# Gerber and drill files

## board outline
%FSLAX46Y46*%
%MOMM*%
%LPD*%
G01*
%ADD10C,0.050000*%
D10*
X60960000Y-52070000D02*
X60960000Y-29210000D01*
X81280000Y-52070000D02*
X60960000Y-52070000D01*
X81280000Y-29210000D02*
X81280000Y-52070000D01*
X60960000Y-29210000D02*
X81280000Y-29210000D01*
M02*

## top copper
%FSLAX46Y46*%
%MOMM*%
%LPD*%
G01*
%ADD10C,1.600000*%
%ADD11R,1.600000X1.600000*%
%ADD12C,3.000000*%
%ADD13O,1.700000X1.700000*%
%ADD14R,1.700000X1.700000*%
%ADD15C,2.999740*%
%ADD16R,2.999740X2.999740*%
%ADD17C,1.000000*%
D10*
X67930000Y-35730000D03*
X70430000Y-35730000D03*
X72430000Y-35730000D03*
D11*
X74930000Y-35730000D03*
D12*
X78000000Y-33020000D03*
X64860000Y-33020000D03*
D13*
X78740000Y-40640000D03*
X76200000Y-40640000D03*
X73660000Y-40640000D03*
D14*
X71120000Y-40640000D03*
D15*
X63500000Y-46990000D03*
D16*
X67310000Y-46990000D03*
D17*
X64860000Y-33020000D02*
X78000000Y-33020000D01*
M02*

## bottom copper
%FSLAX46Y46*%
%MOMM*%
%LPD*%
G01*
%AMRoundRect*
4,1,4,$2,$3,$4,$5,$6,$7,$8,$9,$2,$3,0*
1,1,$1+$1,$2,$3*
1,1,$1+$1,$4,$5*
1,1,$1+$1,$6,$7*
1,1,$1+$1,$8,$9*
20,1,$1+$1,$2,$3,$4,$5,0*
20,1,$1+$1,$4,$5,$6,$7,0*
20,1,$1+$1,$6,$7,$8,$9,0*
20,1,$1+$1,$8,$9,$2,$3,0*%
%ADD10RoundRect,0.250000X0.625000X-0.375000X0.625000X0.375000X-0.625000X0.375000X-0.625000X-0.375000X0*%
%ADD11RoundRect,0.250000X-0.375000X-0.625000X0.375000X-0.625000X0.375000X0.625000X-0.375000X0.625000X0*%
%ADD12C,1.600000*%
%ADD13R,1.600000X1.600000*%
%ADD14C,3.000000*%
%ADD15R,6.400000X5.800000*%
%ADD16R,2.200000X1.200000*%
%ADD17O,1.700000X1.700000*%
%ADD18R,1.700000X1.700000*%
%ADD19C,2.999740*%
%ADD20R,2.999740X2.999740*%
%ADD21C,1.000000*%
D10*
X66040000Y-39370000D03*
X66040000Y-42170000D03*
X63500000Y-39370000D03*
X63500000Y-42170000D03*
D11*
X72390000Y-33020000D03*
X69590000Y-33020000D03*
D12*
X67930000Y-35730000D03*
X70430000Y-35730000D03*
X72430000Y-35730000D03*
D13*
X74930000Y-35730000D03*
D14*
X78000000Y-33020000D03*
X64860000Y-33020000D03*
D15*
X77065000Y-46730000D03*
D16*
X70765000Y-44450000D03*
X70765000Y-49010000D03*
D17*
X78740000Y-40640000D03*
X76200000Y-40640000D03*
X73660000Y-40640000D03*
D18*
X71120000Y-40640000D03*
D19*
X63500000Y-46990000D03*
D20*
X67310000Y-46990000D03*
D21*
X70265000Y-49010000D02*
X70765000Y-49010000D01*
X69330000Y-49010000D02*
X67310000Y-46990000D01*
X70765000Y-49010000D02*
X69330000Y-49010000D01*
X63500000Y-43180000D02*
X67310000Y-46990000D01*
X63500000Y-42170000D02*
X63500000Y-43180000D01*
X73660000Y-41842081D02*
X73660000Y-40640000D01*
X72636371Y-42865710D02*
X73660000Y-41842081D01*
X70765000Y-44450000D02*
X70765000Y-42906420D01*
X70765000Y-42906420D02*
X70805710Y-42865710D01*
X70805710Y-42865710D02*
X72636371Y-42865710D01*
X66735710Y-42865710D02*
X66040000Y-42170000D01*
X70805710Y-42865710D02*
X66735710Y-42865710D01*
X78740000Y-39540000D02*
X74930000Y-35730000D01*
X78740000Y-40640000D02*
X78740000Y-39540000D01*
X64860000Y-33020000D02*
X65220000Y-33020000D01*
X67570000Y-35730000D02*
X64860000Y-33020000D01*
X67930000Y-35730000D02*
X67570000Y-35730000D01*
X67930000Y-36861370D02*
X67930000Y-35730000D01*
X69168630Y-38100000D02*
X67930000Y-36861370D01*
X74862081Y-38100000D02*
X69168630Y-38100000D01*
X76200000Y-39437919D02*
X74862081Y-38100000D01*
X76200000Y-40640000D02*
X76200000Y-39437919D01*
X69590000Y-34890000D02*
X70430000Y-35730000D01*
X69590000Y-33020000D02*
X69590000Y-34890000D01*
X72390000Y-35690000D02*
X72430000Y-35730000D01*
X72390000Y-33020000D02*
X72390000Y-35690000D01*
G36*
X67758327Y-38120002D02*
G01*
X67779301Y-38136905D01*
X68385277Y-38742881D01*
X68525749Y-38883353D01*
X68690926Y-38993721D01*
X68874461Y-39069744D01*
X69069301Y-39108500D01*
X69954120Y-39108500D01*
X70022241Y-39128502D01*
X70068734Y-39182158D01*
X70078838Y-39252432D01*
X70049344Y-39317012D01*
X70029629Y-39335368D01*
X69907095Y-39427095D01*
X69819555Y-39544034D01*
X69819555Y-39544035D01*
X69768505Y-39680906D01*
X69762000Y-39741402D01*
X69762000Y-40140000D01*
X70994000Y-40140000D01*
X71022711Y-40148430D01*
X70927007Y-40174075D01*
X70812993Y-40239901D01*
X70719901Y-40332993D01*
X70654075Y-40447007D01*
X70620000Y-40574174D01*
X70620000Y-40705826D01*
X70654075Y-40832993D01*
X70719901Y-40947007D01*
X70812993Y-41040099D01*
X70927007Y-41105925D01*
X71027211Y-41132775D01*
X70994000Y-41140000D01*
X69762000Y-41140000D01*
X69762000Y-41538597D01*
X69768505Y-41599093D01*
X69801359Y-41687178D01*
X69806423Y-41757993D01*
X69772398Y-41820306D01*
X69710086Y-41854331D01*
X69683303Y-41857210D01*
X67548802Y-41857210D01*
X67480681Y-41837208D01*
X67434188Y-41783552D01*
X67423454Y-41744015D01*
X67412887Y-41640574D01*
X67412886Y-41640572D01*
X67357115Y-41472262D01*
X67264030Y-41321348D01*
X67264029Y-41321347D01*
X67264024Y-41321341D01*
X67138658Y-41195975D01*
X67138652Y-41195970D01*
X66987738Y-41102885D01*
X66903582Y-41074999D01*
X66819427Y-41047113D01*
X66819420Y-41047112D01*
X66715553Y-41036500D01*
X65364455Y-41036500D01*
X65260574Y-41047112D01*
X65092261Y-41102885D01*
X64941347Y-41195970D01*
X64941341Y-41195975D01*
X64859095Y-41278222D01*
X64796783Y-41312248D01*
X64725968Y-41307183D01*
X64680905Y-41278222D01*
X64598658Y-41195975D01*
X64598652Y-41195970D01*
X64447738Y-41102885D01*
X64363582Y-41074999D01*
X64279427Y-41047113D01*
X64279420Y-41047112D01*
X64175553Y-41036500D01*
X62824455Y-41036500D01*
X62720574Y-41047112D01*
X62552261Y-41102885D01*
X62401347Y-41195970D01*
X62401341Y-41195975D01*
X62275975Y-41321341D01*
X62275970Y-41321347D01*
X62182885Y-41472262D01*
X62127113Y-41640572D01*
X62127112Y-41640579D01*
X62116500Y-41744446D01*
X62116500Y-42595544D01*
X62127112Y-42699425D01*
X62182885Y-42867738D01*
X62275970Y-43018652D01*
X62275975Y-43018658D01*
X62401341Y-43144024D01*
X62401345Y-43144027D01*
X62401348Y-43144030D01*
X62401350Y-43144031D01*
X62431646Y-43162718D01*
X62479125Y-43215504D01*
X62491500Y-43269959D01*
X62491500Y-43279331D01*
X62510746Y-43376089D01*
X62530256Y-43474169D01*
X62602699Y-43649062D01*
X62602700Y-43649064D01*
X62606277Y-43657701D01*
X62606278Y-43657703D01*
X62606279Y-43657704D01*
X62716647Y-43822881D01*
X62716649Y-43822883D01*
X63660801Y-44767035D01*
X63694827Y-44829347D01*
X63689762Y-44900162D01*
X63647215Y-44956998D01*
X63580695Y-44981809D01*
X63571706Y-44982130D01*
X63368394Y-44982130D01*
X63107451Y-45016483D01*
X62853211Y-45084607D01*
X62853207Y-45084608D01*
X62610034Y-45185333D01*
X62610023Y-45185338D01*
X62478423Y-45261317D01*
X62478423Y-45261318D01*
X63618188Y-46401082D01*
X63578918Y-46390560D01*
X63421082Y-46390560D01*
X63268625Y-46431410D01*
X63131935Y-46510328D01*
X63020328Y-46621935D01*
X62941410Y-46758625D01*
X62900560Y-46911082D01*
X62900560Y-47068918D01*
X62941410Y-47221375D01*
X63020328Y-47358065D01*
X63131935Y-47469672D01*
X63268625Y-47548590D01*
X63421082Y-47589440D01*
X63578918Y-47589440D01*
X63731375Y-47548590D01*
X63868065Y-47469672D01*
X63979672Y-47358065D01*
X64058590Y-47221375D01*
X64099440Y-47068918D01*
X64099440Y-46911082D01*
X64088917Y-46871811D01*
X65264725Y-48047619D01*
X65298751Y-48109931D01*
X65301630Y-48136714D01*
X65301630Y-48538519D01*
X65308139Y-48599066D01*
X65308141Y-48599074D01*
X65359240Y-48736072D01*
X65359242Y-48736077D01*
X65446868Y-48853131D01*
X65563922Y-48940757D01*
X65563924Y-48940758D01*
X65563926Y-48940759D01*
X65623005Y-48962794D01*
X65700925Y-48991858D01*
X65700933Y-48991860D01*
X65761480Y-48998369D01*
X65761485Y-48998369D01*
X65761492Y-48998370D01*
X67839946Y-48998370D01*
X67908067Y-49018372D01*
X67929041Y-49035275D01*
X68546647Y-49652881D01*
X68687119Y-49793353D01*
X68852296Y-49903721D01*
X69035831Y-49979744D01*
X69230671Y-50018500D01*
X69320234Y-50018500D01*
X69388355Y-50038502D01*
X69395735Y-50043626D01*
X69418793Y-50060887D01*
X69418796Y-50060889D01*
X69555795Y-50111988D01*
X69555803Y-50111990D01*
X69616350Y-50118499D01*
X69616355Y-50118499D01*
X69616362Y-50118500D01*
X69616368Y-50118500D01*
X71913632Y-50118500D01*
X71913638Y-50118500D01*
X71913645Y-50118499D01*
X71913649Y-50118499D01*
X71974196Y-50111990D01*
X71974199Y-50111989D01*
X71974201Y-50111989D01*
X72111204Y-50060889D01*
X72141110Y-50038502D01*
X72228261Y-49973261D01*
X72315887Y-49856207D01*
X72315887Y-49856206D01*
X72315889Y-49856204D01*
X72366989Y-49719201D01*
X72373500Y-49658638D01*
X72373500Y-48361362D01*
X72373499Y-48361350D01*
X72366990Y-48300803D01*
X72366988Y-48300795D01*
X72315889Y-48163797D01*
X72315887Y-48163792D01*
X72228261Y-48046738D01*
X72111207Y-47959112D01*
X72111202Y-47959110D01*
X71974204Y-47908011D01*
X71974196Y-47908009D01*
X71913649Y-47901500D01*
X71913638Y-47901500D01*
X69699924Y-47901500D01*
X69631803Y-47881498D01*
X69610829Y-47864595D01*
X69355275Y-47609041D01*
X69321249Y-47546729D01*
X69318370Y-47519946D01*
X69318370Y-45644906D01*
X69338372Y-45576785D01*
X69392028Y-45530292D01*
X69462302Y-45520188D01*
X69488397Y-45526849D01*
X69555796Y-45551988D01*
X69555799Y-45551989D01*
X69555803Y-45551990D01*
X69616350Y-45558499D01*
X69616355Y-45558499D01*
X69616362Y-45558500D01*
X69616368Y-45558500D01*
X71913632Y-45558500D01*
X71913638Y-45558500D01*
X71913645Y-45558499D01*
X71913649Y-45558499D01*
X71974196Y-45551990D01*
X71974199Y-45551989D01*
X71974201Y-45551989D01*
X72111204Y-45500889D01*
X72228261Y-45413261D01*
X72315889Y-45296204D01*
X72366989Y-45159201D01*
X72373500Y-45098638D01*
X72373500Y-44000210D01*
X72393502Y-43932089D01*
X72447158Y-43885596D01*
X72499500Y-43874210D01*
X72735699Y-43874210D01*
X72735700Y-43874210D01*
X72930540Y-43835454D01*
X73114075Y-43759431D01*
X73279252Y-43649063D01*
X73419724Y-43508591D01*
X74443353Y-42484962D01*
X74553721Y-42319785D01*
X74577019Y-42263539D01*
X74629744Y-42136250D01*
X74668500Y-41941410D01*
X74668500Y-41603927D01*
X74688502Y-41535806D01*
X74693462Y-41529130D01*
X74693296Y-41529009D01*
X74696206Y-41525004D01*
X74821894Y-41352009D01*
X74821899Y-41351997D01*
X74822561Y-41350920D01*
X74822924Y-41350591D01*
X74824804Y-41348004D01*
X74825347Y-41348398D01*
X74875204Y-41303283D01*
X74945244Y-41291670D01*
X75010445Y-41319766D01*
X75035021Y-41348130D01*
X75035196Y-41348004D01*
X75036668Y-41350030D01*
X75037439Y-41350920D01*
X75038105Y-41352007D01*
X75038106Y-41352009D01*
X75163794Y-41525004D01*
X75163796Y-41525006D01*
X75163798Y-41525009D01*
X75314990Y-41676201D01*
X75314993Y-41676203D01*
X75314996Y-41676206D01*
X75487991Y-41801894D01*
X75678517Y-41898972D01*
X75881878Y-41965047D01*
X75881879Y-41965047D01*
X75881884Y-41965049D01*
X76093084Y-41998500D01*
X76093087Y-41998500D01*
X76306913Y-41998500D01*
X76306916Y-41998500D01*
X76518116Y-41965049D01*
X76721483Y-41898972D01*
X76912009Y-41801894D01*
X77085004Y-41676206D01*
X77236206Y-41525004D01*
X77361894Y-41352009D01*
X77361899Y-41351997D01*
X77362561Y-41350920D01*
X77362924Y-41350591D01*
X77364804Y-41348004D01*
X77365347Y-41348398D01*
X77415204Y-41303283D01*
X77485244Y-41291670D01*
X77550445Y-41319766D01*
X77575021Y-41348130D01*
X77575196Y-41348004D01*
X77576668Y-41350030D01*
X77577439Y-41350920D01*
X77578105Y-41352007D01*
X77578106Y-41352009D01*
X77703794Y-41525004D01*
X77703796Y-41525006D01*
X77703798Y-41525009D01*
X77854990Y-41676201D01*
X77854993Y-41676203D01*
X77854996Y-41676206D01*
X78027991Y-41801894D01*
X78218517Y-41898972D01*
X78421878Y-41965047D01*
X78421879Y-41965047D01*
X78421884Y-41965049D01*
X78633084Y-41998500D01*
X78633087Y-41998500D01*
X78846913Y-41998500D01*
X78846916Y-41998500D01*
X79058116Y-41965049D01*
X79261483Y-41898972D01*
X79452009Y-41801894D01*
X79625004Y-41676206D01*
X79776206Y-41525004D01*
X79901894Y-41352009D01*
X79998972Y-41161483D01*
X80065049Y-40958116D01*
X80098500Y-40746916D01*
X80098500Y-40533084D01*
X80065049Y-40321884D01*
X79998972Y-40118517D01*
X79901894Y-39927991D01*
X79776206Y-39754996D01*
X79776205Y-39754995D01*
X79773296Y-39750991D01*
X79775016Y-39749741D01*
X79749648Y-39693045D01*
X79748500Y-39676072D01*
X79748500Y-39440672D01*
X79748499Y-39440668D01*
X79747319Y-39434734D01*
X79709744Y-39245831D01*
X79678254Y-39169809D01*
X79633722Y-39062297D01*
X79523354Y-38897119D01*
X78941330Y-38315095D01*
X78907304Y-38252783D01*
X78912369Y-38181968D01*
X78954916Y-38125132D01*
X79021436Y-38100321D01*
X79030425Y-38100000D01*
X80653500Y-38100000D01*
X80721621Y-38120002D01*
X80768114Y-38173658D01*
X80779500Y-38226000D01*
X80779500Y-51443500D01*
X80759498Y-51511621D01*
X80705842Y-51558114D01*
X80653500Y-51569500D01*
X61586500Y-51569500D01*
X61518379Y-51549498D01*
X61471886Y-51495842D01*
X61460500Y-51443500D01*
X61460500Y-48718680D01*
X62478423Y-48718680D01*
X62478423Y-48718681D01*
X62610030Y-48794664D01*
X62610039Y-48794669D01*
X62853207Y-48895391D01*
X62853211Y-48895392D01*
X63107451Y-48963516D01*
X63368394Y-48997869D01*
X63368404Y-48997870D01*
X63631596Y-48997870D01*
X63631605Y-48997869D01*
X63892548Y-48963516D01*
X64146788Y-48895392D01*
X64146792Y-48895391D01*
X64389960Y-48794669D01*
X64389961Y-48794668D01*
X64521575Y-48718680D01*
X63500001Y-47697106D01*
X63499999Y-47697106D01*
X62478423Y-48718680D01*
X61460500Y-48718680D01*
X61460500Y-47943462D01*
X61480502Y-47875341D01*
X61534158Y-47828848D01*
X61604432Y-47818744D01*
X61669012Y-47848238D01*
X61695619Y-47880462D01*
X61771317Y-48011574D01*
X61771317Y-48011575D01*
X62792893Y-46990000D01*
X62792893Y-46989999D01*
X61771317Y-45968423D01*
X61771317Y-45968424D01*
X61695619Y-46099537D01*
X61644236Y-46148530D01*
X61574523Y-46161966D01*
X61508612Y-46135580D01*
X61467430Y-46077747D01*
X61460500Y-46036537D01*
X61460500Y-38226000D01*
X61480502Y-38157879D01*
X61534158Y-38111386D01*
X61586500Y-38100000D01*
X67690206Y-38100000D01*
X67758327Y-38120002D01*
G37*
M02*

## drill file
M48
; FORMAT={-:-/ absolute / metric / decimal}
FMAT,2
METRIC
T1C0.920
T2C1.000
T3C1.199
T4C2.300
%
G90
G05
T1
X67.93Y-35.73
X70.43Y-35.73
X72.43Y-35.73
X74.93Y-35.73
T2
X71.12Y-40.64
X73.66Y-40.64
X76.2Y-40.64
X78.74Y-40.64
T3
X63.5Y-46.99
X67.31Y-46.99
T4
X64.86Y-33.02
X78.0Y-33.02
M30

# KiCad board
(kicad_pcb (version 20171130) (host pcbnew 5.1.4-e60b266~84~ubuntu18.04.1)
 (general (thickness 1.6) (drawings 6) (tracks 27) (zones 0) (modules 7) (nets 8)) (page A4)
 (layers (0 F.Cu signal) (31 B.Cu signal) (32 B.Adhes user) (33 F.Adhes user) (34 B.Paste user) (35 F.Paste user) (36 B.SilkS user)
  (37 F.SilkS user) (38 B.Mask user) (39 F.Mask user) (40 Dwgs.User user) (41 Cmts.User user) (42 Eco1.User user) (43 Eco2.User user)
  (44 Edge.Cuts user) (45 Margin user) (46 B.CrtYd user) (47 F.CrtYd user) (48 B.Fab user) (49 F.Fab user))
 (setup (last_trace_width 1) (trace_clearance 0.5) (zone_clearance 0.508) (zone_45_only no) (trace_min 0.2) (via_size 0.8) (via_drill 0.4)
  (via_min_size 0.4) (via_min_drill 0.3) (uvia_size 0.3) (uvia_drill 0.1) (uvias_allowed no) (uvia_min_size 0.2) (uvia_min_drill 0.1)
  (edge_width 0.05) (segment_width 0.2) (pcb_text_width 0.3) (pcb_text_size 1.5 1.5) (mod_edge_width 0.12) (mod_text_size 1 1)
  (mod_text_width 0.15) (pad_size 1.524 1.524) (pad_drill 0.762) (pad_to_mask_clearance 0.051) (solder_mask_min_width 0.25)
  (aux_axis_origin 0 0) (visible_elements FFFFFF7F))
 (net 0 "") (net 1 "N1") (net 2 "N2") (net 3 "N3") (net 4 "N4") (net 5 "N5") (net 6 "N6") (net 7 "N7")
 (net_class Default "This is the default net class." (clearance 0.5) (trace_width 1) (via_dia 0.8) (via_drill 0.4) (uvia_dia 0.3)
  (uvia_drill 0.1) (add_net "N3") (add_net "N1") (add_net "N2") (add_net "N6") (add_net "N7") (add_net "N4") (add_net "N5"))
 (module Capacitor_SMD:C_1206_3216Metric (layer B.Cu) (at 66.04 40.77 90)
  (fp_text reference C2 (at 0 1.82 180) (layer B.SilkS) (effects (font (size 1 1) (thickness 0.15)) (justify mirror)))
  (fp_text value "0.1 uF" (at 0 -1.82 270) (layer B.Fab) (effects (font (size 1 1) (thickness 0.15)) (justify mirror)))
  (pad 2 smd roundrect (at 1.4 0 90) (size 1.25 1.75) (layers B.Cu B.Paste B.Mask) (roundrect_rratio 0.2) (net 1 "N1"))
  (pad 1 smd roundrect (at -1.4 0 90) (size 1.25 1.75) (layers B.Cu B.Paste B.Mask) (roundrect_rratio 0.2) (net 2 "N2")))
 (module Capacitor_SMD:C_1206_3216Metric (layer B.Cu) (at 63.5 40.77 90)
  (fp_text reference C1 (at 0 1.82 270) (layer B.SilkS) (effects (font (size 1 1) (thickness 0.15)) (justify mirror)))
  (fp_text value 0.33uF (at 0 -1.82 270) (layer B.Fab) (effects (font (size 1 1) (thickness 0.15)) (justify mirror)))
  (pad 2 smd roundrect (at 1.4 0 90) (size 1.25 1.75) (layers B.Cu B.Paste B.Mask) (roundrect_rratio 0.2) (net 1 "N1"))
  (pad 1 smd roundrect (at -1.4 0 90) (size 1.25 1.75) (layers B.Cu B.Paste B.Mask) (roundrect_rratio 0.2) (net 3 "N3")))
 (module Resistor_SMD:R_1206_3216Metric (layer B.Cu) (at 70.99 33.02)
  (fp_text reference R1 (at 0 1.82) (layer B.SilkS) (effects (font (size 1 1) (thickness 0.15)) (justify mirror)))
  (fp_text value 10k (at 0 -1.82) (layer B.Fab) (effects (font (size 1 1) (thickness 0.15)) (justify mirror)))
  (pad 2 smd roundrect (at 1.4 0) (size 1.25 1.75) (layers B.Cu B.Paste B.Mask) (roundrect_rratio 0.2) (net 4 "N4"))
  (pad 1 smd roundrect (at -1.4 0) (size 1.25 1.75) (layers B.Cu B.Paste B.Mask) (roundrect_rratio 0.2) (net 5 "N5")))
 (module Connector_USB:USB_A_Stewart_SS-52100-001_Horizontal (layer F.Cu) (at 74.93 35.73 180)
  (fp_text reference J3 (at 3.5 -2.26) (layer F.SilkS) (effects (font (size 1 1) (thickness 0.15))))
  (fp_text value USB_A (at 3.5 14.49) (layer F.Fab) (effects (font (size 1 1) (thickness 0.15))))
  (pad 4 thru_hole circle (at 7 0 180) (size 1.6 1.6) (drill 0.92) (layers *.Cu *.Mask) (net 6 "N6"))
  (pad 3 thru_hole circle (at 4.5 0 180) (size 1.6 1.6) (drill 0.92) (layers *.Cu *.Mask) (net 5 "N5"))
  (pad 2 thru_hole circle (at 2.5 0 180) (size 1.6 1.6) (drill 0.92) (layers *.Cu *.Mask) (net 4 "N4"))
  (pad 1 thru_hole rect (at 0 0 180) (size 1.6 1.6) (drill 0.92) (layers *.Cu *.Mask) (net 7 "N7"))
  (pad 5 thru_hole circle (at -3.07 2.71 180) (size 3 3) (drill 2.3) (layers *.Cu *.Mask) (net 6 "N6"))
  (pad 5 thru_hole circle (at 10.07 2.71 180) (size 3 3) (drill 2.3) (layers *.Cu *.Mask) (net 6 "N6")))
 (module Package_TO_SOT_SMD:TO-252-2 (layer B.Cu) (at 74.965 46.73)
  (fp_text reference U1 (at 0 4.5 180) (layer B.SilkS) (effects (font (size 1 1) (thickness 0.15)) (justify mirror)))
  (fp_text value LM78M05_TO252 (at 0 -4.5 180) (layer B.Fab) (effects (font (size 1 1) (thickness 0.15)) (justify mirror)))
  (pad "" smd rect (at 0.425 -1.525) (size 3.05 2.75) (layers B.Paste))
  (pad "" smd rect (at 3.775 1.525) (size 3.05 2.75) (layers B.Paste))
  (pad "" smd rect (at 0.425 1.525) (size 3.05 2.75) (layers B.Paste))
  (pad "" smd rect (at 3.775 -1.525) (size 3.05 2.75) (layers B.Paste))
  (pad 2 smd rect (at 2.1 0) (size 6.4 5.8) (layers B.Cu B.Mask) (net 1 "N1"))
  (pad 3 smd rect (at -4.2 -2.28) (size 2.2 1.2) (layers B.Cu B.Paste B.Mask) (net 2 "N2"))
  (pad 1 smd rect (at -4.2 2.28) (size 2.2 1.2) (layers B.Cu B.Paste B.Mask) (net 3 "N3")))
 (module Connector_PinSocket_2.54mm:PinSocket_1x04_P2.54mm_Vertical (layer F.Cu) (at 71.12 40.64 90)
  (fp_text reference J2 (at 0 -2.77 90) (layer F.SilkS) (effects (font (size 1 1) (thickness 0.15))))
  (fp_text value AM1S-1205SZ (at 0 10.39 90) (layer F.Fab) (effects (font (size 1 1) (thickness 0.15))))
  (pad 4 thru_hole oval (at 0 7.62 90) (size 1.7 1.7) (drill 1) (layers *.Cu *.Mask) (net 7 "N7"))
  (pad 3 thru_hole oval (at 0 5.08 90) (size 1.7 1.7) (drill 1) (layers *.Cu *.Mask) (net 6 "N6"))
  (pad 2 thru_hole oval (at 0 2.54 90) (size 1.7 1.7) (drill 1) (layers *.Cu *.Mask) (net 2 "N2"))
  (pad 1 thru_hole rect (at 0 0 90) (size 1.7 1.7) (drill 1) (layers *.Cu *.Mask) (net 1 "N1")))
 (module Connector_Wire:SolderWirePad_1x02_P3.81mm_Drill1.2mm (layer F.Cu) (at 67.31 46.99 180)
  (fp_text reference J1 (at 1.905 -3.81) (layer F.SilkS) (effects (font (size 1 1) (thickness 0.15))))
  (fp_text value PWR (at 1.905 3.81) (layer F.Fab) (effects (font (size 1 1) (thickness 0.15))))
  (pad 2 thru_hole circle (at 3.81 0 180) (size 2.99974 2.99974) (drill 1.19888) (layers *.Cu *.Mask) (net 1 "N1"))
  (pad 1 thru_hole rect (at 0 0 180) (size 2.99974 2.99974) (drill 1.19888) (layers *.Cu *.Mask) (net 3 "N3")))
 (gr_line (start 60.96 52.07) (end 60.96 29.21) (layer Edge.Cuts) (width 0.05))
 (gr_line (start 81.28 52.07) (end 60.96 52.07) (layer Edge.Cuts) (width 0.05))
 (gr_line (start 81.28 29.21) (end 81.28 52.07) (layer Edge.Cuts) (width 0.05))
 (gr_line (start 60.96 29.21) (end 81.28 29.21) (layer Edge.Cuts) (width 0.05))
 (segment (start 70.265 49.01) (end 70.765 49.01) (width 1) (layer B.Cu) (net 3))
 (segment (start 69.33 49.01) (end 67.31 46.99) (width 1) (layer B.Cu) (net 3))
 (segment (start 70.765 49.01) (end 69.33 49.01) (width 1) (layer B.Cu) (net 3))
 (segment (start 63.5 43.18) (end 67.31 46.99) (width 1) (layer B.Cu) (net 3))
 (segment (start 63.5 42.17) (end 63.5 43.18) (width 1) (layer B.Cu) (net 3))
 (segment (start 73.66 41.842081) (end 73.66 40.64) (width 1) (layer B.Cu) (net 2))
 (segment (start 72.636371 42.86571) (end 73.66 41.842081) (width 1) (layer B.Cu) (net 2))
 (segment (start 70.765 44.45) (end 70.765 42.90642) (width 1) (layer B.Cu) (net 2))
 (segment (start 70.765 42.90642) (end 70.80571 42.86571) (width 1) (layer B.Cu) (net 2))
 (segment (start 70.80571 42.86571) (end 72.636371 42.86571) (width 1) (layer B.Cu) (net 2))
 (segment (start 66.73571 42.86571) (end 66.04 42.17) (width 1) (layer B.Cu) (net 2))
 (segment (start 70.80571 42.86571) (end 66.73571 42.86571) (width 1) (layer B.Cu) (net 2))
 (segment (start 78.74 39.54) (end 74.93 35.73) (width 1) (layer B.Cu) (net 7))
 (segment (start 78.74 40.64) (end 78.74 39.54) (width 1) (layer B.Cu) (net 7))
 (segment (start 64.86 33.02) (end 78 33.02) (width 1) (layer F.Cu) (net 6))
 (segment (start 64.86 33.02) (end 65.22 33.02) (width 1) (layer B.Cu) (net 6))
 (segment (start 67.57 35.73) (end 64.86 33.02) (width 1) (layer B.Cu) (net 6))
 (segment (start 67.93 35.73) (end 67.57 35.73) (width 1) (layer B.Cu) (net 6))
 (segment (start 67.93 36.86137) (end 67.93 35.73) (width 1) (layer B.Cu) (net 6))
 (segment (start 69.16863 38.1) (end 67.93 36.86137) (width 1) (layer B.Cu) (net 6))
 (segment (start 74.862081 38.1) (end 69.16863 38.1) (width 1) (layer B.Cu) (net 6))
 (segment (start 76.2 39.437919) (end 74.862081 38.1) (width 1) (layer B.Cu) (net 6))
 (segment (start 76.2 40.64) (end 76.2 39.437919) (width 1) (layer B.Cu) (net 6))
 (segment (start 69.59 34.89) (end 70.43 35.73) (width 1) (layer B.Cu) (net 5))
 (segment (start 69.59 33.02) (end 69.59 34.89) (width 1) (layer B.Cu) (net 5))
 (segment (start 72.39 35.69) (end 72.43 35.73) (width 1) (layer B.Cu) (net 4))
 (segment (start 72.39 33.02) (end 72.39 35.69) (width 1) (layer B.Cu) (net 4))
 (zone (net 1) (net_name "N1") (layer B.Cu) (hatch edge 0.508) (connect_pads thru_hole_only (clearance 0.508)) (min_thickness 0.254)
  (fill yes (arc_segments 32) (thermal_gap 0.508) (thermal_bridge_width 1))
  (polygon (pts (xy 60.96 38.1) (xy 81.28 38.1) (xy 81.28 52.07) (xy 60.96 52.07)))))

